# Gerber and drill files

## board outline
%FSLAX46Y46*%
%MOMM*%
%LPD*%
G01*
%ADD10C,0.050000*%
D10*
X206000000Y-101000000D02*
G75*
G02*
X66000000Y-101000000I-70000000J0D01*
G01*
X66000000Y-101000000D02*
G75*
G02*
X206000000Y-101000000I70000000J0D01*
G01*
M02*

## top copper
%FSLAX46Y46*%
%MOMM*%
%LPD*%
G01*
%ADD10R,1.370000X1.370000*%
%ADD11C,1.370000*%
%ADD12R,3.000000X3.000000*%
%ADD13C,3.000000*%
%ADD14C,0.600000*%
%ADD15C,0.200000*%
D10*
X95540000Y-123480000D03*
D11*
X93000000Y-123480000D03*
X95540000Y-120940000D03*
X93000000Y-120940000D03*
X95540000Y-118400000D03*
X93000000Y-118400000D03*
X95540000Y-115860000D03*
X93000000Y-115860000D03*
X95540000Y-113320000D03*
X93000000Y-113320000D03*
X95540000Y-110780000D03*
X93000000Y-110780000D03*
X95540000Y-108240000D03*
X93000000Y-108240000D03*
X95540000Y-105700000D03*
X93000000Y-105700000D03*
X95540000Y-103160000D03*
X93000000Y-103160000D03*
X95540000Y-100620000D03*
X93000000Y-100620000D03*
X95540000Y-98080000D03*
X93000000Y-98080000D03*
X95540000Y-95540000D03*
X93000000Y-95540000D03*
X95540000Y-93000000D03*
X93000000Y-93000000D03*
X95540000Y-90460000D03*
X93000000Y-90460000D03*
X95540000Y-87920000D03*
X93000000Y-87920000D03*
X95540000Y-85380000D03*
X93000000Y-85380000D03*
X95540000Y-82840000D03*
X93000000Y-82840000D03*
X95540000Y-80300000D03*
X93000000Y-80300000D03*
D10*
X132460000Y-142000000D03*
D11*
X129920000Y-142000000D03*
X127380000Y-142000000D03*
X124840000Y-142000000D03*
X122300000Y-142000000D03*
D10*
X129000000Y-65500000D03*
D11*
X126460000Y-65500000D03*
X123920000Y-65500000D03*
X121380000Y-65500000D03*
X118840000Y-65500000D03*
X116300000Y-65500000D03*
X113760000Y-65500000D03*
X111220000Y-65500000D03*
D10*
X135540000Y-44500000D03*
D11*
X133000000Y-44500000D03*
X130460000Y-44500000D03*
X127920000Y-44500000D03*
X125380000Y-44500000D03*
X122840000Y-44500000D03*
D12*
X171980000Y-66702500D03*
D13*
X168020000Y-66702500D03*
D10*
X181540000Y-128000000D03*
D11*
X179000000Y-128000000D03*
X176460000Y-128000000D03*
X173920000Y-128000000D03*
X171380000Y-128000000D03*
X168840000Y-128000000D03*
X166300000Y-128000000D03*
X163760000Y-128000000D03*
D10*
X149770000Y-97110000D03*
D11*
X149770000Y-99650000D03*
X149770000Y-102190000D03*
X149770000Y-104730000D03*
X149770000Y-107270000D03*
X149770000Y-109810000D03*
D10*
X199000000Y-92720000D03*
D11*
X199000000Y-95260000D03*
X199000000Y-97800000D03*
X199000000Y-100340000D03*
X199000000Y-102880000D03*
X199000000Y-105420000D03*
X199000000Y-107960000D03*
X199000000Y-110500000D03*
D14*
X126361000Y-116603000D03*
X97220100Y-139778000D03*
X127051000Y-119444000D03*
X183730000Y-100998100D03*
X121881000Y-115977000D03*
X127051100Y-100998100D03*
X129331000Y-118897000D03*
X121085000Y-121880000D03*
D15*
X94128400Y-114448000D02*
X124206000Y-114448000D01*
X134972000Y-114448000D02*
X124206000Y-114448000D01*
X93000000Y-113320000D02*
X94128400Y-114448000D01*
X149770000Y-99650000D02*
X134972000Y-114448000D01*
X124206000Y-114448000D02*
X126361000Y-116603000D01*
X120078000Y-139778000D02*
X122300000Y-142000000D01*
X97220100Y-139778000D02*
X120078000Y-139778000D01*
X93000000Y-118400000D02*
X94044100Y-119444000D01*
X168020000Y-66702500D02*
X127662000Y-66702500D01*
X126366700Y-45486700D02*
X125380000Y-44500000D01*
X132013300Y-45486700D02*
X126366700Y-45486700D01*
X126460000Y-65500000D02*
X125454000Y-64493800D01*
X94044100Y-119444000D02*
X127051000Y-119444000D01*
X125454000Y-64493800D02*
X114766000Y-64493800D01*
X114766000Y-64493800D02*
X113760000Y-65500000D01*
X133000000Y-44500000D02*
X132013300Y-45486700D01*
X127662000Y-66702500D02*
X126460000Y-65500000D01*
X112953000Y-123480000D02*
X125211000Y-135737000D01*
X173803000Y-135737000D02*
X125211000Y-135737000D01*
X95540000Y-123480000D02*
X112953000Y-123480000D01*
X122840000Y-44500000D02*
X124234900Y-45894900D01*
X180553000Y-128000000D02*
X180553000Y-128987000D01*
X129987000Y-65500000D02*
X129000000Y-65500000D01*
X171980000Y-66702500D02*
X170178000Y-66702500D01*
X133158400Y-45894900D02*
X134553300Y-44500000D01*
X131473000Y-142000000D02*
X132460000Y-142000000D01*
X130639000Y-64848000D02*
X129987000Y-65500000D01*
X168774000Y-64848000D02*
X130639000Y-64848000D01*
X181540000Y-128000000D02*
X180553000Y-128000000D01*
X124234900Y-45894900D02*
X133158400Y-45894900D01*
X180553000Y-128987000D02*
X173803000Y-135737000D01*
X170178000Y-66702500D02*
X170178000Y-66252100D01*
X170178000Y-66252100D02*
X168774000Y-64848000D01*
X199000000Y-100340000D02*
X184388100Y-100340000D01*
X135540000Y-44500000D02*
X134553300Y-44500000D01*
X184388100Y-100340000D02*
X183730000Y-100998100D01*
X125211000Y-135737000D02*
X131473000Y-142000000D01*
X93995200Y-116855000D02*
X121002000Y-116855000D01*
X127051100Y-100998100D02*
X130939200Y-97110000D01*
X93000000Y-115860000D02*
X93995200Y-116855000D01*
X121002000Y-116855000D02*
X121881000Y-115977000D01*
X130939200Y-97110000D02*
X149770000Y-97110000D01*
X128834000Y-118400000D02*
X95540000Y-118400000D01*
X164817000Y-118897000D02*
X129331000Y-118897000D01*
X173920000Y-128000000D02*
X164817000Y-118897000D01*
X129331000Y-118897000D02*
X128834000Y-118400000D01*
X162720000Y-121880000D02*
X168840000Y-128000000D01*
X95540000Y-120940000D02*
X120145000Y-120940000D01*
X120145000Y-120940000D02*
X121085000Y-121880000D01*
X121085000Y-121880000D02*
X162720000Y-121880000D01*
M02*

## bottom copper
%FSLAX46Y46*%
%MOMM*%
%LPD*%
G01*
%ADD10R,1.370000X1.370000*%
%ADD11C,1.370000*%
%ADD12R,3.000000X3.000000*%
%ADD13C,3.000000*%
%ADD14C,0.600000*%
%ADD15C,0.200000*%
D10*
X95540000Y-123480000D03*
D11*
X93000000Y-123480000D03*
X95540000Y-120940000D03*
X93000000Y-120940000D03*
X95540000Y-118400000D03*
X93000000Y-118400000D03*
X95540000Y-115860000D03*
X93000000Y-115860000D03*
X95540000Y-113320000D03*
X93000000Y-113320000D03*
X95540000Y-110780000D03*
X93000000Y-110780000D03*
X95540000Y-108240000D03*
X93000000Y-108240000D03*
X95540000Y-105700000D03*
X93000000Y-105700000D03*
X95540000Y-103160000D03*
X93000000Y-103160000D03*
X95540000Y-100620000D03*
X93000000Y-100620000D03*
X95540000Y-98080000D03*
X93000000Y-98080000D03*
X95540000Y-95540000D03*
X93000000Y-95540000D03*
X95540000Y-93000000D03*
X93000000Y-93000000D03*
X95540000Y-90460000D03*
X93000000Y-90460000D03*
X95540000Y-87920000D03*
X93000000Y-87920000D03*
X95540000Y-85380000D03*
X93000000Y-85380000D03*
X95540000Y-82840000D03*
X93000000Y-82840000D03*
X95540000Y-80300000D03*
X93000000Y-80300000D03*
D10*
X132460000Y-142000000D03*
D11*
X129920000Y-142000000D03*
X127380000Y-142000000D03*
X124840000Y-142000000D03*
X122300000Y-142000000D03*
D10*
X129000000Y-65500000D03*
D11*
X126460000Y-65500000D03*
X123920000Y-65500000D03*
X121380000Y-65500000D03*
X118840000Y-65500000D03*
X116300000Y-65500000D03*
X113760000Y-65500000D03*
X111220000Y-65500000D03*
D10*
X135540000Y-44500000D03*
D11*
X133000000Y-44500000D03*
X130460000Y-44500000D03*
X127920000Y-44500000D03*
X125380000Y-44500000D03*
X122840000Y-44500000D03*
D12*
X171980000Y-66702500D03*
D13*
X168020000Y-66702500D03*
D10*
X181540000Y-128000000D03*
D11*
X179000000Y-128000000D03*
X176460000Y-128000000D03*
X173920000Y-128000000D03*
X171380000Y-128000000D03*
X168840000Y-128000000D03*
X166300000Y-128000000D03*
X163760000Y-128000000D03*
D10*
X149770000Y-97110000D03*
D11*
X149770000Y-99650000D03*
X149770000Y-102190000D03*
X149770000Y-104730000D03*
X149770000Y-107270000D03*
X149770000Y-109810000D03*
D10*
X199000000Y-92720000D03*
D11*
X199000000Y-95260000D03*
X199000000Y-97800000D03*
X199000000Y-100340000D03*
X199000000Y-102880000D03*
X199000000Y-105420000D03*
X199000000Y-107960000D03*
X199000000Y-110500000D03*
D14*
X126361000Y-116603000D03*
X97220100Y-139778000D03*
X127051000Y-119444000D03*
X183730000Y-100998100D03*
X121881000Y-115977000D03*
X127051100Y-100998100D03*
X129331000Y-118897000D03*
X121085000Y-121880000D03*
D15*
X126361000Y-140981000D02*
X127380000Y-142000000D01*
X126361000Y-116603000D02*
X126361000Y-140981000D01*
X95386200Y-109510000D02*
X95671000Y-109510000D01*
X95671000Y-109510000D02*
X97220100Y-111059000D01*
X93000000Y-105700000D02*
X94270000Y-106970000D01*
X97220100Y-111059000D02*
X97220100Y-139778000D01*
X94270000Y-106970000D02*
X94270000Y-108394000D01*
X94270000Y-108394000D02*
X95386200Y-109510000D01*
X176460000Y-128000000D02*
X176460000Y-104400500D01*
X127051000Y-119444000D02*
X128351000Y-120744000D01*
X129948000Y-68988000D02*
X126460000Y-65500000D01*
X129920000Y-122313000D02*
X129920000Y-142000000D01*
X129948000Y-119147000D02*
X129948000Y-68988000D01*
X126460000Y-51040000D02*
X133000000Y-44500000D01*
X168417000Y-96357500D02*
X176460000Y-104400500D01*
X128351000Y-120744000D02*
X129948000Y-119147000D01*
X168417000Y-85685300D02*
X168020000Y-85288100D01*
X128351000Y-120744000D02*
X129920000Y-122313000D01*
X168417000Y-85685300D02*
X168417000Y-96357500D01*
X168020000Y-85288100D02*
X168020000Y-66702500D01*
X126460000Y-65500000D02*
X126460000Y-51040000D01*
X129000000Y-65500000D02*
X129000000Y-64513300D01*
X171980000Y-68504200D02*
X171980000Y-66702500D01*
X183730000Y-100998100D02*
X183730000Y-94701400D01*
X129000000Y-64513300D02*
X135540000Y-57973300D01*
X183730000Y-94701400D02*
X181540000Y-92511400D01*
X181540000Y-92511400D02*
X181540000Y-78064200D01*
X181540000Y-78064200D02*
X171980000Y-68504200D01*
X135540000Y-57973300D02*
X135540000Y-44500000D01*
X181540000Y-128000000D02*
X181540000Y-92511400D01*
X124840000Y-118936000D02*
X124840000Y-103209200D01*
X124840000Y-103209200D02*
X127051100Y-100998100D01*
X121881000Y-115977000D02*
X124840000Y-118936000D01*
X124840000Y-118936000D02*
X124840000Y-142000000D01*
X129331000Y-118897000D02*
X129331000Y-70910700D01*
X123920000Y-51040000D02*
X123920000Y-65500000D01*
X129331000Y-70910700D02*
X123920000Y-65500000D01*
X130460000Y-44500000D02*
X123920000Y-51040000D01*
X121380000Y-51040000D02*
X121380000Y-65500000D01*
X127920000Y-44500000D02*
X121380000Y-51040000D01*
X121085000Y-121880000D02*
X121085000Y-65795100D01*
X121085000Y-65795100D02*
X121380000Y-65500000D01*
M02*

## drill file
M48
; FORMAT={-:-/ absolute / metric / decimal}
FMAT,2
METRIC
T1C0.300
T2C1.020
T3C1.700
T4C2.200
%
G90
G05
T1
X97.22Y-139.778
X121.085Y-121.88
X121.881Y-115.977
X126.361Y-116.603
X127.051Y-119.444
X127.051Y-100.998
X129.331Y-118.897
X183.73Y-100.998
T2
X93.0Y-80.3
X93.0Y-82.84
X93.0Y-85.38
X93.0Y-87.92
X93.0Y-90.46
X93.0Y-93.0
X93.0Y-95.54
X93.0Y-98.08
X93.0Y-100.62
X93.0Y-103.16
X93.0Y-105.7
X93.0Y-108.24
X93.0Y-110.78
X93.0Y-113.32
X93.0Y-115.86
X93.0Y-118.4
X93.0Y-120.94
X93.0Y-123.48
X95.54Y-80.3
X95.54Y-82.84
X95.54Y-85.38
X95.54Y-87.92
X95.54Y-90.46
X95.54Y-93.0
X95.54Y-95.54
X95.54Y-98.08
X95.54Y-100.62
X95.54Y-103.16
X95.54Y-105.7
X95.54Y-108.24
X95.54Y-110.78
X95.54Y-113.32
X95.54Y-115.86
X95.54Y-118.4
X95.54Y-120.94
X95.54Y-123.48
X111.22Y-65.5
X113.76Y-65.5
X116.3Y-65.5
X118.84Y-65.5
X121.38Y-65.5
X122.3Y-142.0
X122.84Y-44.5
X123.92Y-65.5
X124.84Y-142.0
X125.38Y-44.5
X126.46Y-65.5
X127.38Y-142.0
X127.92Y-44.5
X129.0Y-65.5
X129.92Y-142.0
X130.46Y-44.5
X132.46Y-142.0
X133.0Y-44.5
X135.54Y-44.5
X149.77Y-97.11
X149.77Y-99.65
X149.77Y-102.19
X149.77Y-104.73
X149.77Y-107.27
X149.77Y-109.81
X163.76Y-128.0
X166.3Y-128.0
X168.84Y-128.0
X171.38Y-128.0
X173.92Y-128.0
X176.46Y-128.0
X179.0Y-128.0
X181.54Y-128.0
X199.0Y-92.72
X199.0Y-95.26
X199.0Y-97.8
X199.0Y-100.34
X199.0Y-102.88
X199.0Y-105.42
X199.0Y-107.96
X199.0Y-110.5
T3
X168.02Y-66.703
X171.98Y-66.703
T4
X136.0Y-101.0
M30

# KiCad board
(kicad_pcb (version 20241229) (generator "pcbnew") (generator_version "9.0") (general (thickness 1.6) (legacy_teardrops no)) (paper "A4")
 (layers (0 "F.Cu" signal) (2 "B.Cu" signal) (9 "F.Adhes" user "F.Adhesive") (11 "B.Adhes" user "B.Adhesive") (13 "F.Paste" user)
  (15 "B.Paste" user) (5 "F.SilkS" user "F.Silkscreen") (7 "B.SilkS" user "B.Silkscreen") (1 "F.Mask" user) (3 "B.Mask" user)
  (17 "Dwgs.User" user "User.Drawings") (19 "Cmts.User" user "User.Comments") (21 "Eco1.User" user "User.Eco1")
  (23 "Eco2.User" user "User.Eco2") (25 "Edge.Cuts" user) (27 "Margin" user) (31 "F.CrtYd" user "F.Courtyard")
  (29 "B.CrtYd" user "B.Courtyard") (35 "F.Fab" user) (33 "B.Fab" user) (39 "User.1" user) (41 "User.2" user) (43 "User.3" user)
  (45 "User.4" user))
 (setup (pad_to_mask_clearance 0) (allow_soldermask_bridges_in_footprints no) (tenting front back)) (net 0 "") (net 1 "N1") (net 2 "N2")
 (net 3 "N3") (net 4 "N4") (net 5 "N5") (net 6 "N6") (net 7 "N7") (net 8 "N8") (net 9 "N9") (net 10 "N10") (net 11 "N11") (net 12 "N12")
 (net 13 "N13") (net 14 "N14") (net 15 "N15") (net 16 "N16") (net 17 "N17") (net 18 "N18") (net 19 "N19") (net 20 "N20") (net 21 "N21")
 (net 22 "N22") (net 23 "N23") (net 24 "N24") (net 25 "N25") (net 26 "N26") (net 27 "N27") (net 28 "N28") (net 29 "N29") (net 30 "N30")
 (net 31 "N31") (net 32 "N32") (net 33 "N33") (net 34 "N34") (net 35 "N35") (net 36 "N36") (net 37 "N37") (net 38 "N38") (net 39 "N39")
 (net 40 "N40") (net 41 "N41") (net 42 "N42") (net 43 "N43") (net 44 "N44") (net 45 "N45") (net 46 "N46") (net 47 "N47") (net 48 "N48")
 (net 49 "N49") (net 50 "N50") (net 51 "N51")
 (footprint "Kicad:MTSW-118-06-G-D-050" (layer "F.Cu") (at 95.54 123.48 90)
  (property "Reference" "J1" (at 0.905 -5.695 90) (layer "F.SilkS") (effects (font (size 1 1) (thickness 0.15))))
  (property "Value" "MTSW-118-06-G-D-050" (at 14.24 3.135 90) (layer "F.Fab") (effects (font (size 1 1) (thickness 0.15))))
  (pad "01" thru_hole rect (at 0 0 90) (size 1.37 1.37) (drill 1.02) (layers "*.Cu" "*.Mask") (remove_unused_layers no) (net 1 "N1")
   (solder_mask_margin 0.102))
  (pad "02" thru_hole circle (at 0 -2.54 90) (size 1.37 1.37) (drill 1.02) (layers "*.Cu" "*.Mask") (remove_unused_layers no) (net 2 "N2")
   (solder_mask_margin 0.102))
  (pad "03" thru_hole circle (at 2.54 0 90) (size 1.37 1.37) (drill 1.02) (layers "*.Cu" "*.Mask") (remove_unused_layers no) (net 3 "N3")
   (solder_mask_margin 0.102))
  (pad "04" thru_hole circle (at 2.54 -2.54 90) (size 1.37 1.37) (drill 1.02) (layers "*.Cu" "*.Mask") (remove_unused_layers no)
   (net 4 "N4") (solder_mask_margin 0.102))
  (pad "05" thru_hole circle (at 5.08 0 90) (size 1.37 1.37) (drill 1.02) (layers "*.Cu" "*.Mask") (remove_unused_layers no) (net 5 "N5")
   (solder_mask_margin 0.102))
  (pad "06" thru_hole circle (at 5.08 -2.54 90) (size 1.37 1.37) (drill 1.02) (layers "*.Cu" "*.Mask") (remove_unused_layers no)
   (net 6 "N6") (solder_mask_margin 0.102))
  (pad "07" thru_hole circle (at 7.62 0 90) (size 1.37 1.37) (drill 1.02) (layers "*.Cu" "*.Mask") (remove_unused_layers no) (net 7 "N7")
   (solder_mask_margin 0.102))
  (pad "08" thru_hole circle (at 7.62 -2.54 90) (size 1.37 1.37) (drill 1.02) (layers "*.Cu" "*.Mask") (remove_unused_layers no)
   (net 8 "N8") (solder_mask_margin 0.102))
  (pad "09" thru_hole circle (at 10.16 0 90) (size 1.37 1.37) (drill 1.02) (layers "*.Cu" "*.Mask") (remove_unused_layers no) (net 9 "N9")
   (solder_mask_margin 0.102))
  (pad "10" thru_hole circle (at 10.16 -2.54 90) (size 1.37 1.37) (drill 1.02) (layers "*.Cu" "*.Mask") (remove_unused_layers no)
   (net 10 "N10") (solder_mask_margin 0.102))
  (pad "11" thru_hole circle (at 12.7 0 90) (size 1.37 1.37) (drill 1.02) (layers "*.Cu" "*.Mask") (remove_unused_layers no) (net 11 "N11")
   (solder_mask_margin 0.102))
  (pad "12" thru_hole circle (at 12.7 -2.54 90) (size 1.37 1.37) (drill 1.02) (layers "*.Cu" "*.Mask") (remove_unused_layers no)
   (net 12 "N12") (solder_mask_margin 0.102))
  (pad "13" thru_hole circle (at 15.24 0 90) (size 1.37 1.37) (drill 1.02) (layers "*.Cu" "*.Mask") (remove_unused_layers no) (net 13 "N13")
   (solder_mask_margin 0.102))
  (pad "14" thru_hole circle (at 15.24 -2.54 90) (size 1.37 1.37) (drill 1.02) (layers "*.Cu" "*.Mask") (remove_unused_layers no)
   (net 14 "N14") (solder_mask_margin 0.102))
  (pad "15" thru_hole circle (at 17.78 0 90) (size 1.37 1.37) (drill 1.02) (layers "*.Cu" "*.Mask") (remove_unused_layers no) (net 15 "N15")
   (solder_mask_margin 0.102))
  (pad "16" thru_hole circle (at 17.78 -2.54 90) (size 1.37 1.37) (drill 1.02) (layers "*.Cu" "*.Mask") (remove_unused_layers no)
   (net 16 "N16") (solder_mask_margin 0.102))
  (pad "17" thru_hole circle (at 20.32 0 90) (size 1.37 1.37) (drill 1.02) (layers "*.Cu" "*.Mask") (remove_unused_layers no) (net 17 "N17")
   (solder_mask_margin 0.102))
  (pad "18" thru_hole circle (at 20.32 -2.54 90) (size 1.37 1.37) (drill 1.02) (layers "*.Cu" "*.Mask") (remove_unused_layers no)
   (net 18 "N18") (solder_mask_margin 0.102))
  (pad "19" thru_hole circle (at 22.86 0 90) (size 1.37 1.37) (drill 1.02) (layers "*.Cu" "*.Mask") (remove_unused_layers no) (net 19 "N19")
   (solder_mask_margin 0.102))
  (pad "20" thru_hole circle (at 22.86 -2.54 90) (size 1.37 1.37) (drill 1.02) (layers "*.Cu" "*.Mask") (remove_unused_layers no)
   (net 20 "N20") (solder_mask_margin 0.102))
  (pad "21" thru_hole circle (at 25.4 0 90) (size 1.37 1.37) (drill 1.02) (layers "*.Cu" "*.Mask") (remove_unused_layers no) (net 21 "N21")
   (solder_mask_margin 0.102))
  (pad "22" thru_hole circle (at 25.4 -2.54 90) (size 1.37 1.37) (drill 1.02) (layers "*.Cu" "*.Mask") (remove_unused_layers no)
   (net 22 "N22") (solder_mask_margin 0.102))
  (pad "23" thru_hole circle (at 27.94 0 90) (size 1.37 1.37) (drill 1.02) (layers "*.Cu" "*.Mask") (remove_unused_layers no) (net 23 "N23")
   (solder_mask_margin 0.102))
  (pad "24" thru_hole circle (at 27.94 -2.54 90) (size 1.37 1.37) (drill 1.02) (layers "*.Cu" "*.Mask") (remove_unused_layers no)
   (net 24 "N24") (solder_mask_margin 0.102))
  (pad "25" thru_hole circle (at 30.48 0 90) (size 1.37 1.37) (drill 1.02) (layers "*.Cu" "*.Mask") (remove_unused_layers no) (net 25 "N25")
   (solder_mask_margin 0.102))
  (pad "26" thru_hole circle (at 30.48 -2.54 90) (size 1.37 1.37) (drill 1.02) (layers "*.Cu" "*.Mask") (remove_unused_layers no)
   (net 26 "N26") (solder_mask_margin 0.102))
  (pad "27" thru_hole circle (at 33.02 0 90) (size 1.37 1.37) (drill 1.02) (layers "*.Cu" "*.Mask") (remove_unused_layers no) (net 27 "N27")
   (solder_mask_margin 0.102))
  (pad "28" thru_hole circle (at 33.02 -2.54 90) (size 1.37 1.37) (drill 1.02) (layers "*.Cu" "*.Mask") (remove_unused_layers no)
   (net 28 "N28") (solder_mask_margin 0.102))
  (pad "29" thru_hole circle (at 35.56 0 90) (size 1.37 1.37) (drill 1.02) (layers "*.Cu" "*.Mask") (remove_unused_layers no) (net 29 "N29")
   (solder_mask_margin 0.102))
  (pad "30" thru_hole circle (at 35.56 -2.54 90) (size 1.37 1.37) (drill 1.02) (layers "*.Cu" "*.Mask") (remove_unused_layers no)
   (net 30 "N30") (solder_mask_margin 0.102))
  (pad "31" thru_hole circle (at 38.1 0 90) (size 1.37 1.37) (drill 1.02) (layers "*.Cu" "*.Mask") (remove_unused_layers no) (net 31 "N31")
   (solder_mask_margin 0.102))
  (pad "32" thru_hole circle (at 38.1 -2.54 90) (size 1.37 1.37) (drill 1.02) (layers "*.Cu" "*.Mask") (remove_unused_layers no)
   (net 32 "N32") (solder_mask_margin 0.102))
  (pad "33" thru_hole circle (at 40.64 0 90) (size 1.37 1.37) (drill 1.02) (layers "*.Cu" "*.Mask") (remove_unused_layers no) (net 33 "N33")
   (solder_mask_margin 0.102))
  (pad "34" thru_hole circle (at 40.64 -2.54 90) (size 1.37 1.37) (drill 1.02) (layers "*.Cu" "*.Mask") (remove_unused_layers no)
   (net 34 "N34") (solder_mask_margin 0.102))
  (pad "35" thru_hole circle (at 43.18 0 90) (size 1.37 1.37) (drill 1.02) (layers "*.Cu" "*.Mask") (remove_unused_layers no) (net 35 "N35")
   (solder_mask_margin 0.102))
  (pad "36" thru_hole circle (at 43.18 -2.54 90) (size 1.37 1.37) (drill 1.02) (layers "*.Cu" "*.Mask") (remove_unused_layers no)
   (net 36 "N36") (solder_mask_margin 0.102)))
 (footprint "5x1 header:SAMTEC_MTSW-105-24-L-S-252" (layer "F.Cu") (at 127.38 142)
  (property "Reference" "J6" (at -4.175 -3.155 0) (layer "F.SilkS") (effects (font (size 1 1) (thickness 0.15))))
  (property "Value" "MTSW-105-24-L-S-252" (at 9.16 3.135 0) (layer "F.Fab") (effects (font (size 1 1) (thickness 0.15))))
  (pad "01" thru_hole rect (at 5.08 0) (size 1.37 1.37) (drill 1.02) (layers "*.Cu" "*.Mask") (remove_unused_layers no) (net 1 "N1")
   (solder_mask_margin 0.102))
  (pad "02" thru_hole circle (at 2.54 0) (size 1.37 1.37) (drill 1.02) (layers "*.Cu" "*.Mask") (remove_unused_layers no) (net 6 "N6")
   (solder_mask_margin 0.102))
  (pad "03" thru_hole circle (at 0 0) (size 1.37 1.37) (drill 1.02) (layers "*.Cu" "*.Mask") (remove_unused_layers no) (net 10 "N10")
   (solder_mask_margin 0.102))
  (pad "04" thru_hole circle (at -2.54 0) (size 1.37 1.37) (drill 1.02) (layers "*.Cu" "*.Mask") (remove_unused_layers no) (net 8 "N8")
   (solder_mask_margin 0.102))
  (pad "05" thru_hole circle (at -5.08 0) (size 1.37 1.37) (drill 1.02) (layers "*.Cu" "*.Mask") (remove_unused_layers no) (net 16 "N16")
   (solder_mask_margin 0.102)))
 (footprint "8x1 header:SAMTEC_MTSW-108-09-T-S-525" (layer "F.Cu") (at 120.11 65.5)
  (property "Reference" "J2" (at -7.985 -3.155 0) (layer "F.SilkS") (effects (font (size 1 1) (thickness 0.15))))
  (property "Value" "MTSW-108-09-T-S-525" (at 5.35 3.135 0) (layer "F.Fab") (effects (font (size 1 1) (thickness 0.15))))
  (pad "01" thru_hole rect (at 8.89 0) (size 1.37 1.37) (drill 1.02) (layers "*.Cu" "*.Mask") (remove_unused_layers no) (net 1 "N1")
   (solder_mask_margin 0.102))
  (pad "02" thru_hole circle (at 6.35 0) (size 1.37 1.37) (drill 1.02) (layers "*.Cu" "*.Mask") (remove_unused_layers no) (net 6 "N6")
   (solder_mask_margin 0.102))
  (pad "03" thru_hole circle (at 3.81 0) (size 1.37 1.37) (drill 1.02) (layers "*.Cu" "*.Mask") (remove_unused_layers no) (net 5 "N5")
   (solder_mask_margin 0.102))
  (pad "04" thru_hole circle (at 1.27 0) (size 1.37 1.37) (drill 1.02) (layers "*.Cu" "*.Mask") (remove_unused_layers no) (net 3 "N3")
   (solder_mask_margin 0.102))
  (pad "05" thru_hole circle (at -1.27 0) (size 1.37 1.37) (drill 1.02) (layers "*.Cu" "*.Mask") (remove_unused_layers no) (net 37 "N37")
   (solder_mask_margin 0.102))
  (pad "06" thru_hole circle (at -3.81 0) (size 1.37 1.37) (drill 1.02) (layers "*.Cu" "*.Mask") (remove_unused_layers no) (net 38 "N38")
   (solder_mask_margin 0.102))
  (pad "07" thru_hole circle (at -6.35 0) (size 1.37 1.37) (drill 1.02) (layers "*.Cu" "*.Mask") (remove_unused_layers no) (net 6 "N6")
   (solder_mask_margin 0.102))
  (pad "08" thru_hole circle (at -8.89 0) (size 1.37 1.37) (drill 1.02) (layers "*.Cu" "*.Mask") (remove_unused_layers no) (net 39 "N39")
   (solder_mask_margin 0.102)))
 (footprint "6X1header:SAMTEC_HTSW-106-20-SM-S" (layer "F.Cu") (at 129.19 44.5)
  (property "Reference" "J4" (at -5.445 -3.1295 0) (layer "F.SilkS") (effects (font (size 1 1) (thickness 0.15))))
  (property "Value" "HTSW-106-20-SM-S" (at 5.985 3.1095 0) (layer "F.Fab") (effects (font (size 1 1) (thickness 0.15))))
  (pad "01" thru_hole rect (at 6.35 0) (size 1.37 1.37) (drill 1.02) (layers "*.Cu" "*.Mask") (remove_unused_layers no) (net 1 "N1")
   (solder_mask_margin 0.102))
  (pad "02" thru_hole circle (at 3.81 0) (size 1.37 1.37) (drill 1.02) (layers "*.Cu" "*.Mask") (remove_unused_layers no) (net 6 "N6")
   (solder_mask_margin 0.102))
  (pad "03" thru_hole circle (at 1.27 0) (size 1.37 1.37) (drill 1.02) (layers "*.Cu" "*.Mask") (remove_unused_layers no) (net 5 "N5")
   (solder_mask_margin 0.102))
  (pad "04" thru_hole circle (at -1.27 0) (size 1.37 1.37) (drill 1.02) (layers "*.Cu" "*.Mask") (remove_unused_layers no) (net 3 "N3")
   (solder_mask_margin 0.102))
  (pad "05" thru_hole circle (at -3.81 0) (size 1.37 1.37) (drill 1.02) (layers "*.Cu" "*.Mask") (remove_unused_layers no) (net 6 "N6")
   (solder_mask_margin 0.102))
  (pad "06" thru_hole circle (at -6.35 0) (size 1.37 1.37) (drill 1.02) (layers "*.Cu" "*.Mask") (remove_unused_layers no) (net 1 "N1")
   (solder_mask_margin 0.102)))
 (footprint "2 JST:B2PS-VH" (layer "F.Cu") (at 170 66.7025 180)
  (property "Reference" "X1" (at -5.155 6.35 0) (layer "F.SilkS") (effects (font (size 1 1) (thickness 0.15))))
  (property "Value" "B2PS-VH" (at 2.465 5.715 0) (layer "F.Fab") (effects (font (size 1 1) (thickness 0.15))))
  (pad "1" thru_hole rect (at -1.98 0 180) (size 3 3) (drill 1.7) (layers "*.Cu" "*.Mask") (remove_unused_layers no) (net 1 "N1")
   (solder_mask_margin 0.102))
  (pad "2" thru_hole circle (at 1.98 0 180) (size 3 3) (drill 1.7) (layers "*.Cu" "*.Mask") (remove_unused_layers no) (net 6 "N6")
   (solder_mask_margin 0.102)))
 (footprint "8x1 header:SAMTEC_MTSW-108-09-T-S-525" (layer "F.Cu") (at 172.65 128)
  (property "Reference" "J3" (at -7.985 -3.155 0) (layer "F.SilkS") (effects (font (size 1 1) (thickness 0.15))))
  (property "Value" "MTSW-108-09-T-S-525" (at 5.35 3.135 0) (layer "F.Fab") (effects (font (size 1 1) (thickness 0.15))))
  (pad "01" thru_hole rect (at 8.89 0) (size 1.37 1.37) (drill 1.02) (layers "*.Cu" "*.Mask") (remove_unused_layers no) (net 1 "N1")
   (solder_mask_margin 0.102))
  (pad "02" thru_hole circle (at 6.35 0) (size 1.37 1.37) (drill 1.02) (layers "*.Cu" "*.Mask") (remove_unused_layers no) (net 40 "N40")
   (solder_mask_margin 0.102))
  (pad "03" thru_hole circle (at 3.81 0) (size 1.37 1.37) (drill 1.02) (layers "*.Cu" "*.Mask") (remove_unused_layers no) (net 6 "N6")
   (solder_mask_margin 0.102))
  (pad "04" thru_hole circle (at 1.27 0) (size 1.37 1.37) (drill 1.02) (layers "*.Cu" "*.Mask") (remove_unused_layers no) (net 5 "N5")
   (solder_mask_margin 0.102))
  (pad "05" thru_hole circle (at -1.27 0) (size 1.37 1.37) (drill 1.02) (layers "*.Cu" "*.Mask") (remove_unused_layers no) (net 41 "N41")
   (solder_mask_margin 0.102))
  (pad "06" thru_hole circle (at -3.81 0) (size 1.37 1.37) (drill 1.02) (layers "*.Cu" "*.Mask") (remove_unused_layers no) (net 3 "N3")
   (solder_mask_margin 0.102))
  (pad "07" thru_hole circle (at -6.35 0) (size 1.37 1.37) (drill 1.02) (layers "*.Cu" "*.Mask") (remove_unused_layers no) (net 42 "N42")
   (solder_mask_margin 0.102))
  (pad "08" thru_hole circle (at -8.89 0) (size 1.37 1.37) (drill 1.02) (layers "*.Cu" "*.Mask") (remove_unused_layers no) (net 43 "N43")
   (solder_mask_margin 0.102)))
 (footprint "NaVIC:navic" (layer "F.Cu") (at 187.77 101.61)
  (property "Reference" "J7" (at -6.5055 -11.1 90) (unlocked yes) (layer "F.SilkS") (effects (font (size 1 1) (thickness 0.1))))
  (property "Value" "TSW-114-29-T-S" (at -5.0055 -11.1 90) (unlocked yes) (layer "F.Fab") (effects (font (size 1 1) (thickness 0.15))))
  (pad "01" thru_hole rect (at -38 -4.5 90) (size 1.37 1.37) (drill 1.02) (layers "*.Cu" "*.Mask") (remove_unused_layers no) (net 8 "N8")
   (solder_mask_margin 0.102))
  (pad "02" thru_hole circle (at -38 -1.96 90) (size 1.37 1.37) (drill 1.02) (layers "*.Cu" "*.Mask") (remove_unused_layers no)
   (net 10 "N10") (solder_mask_margin 0.102))
  (pad "03" thru_hole circle (at -38 0.58 90) (size 1.37 1.37) (drill 1.02) (layers "*.Cu" "*.Mask") (remove_unused_layers no)
   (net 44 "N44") (solder_mask_margin 0.102))
  (pad "04" thru_hole circle (at -38 3.12 90) (size 1.37 1.37) (drill 1.02) (layers "*.Cu" "*.Mask") (remove_unused_layers no)
   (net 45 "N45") (solder_mask_margin 0.102))
  (pad "05" thru_hole circle (at -38 5.66 90) (size 1.37 1.37) (drill 1.02) (layers "*.Cu" "*.Mask") (remove_unused_layers no)
   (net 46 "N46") (solder_mask_margin 0.102))
  (pad "06" thru_hole circle (at -38 8.2 90) (size 1.37 1.37) (drill 1.02) (layers "*.Cu" "*.Mask") (remove_unused_layers no) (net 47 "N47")
   (solder_mask_margin 0.102))
  (pad "7" thru_hole rect (at 11.23 -8.89 90) (size 1.37 1.37) (drill 1.02) (layers "*.Cu" "*.Mask") (remove_unused_layers no)
   (solder_mask_margin 0.102))
  (pad "8" thru_hole circle (at 11.23 -6.35 90) (size 1.37 1.37) (drill 1.02) (layers "*.Cu" "*.Mask") (remove_unused_layers no)
   (solder_mask_margin 0.102))
  (pad "9" thru_hole circle (at 11.23 -3.81 90) (size 1.37 1.37) (drill 1.02) (layers "*.Cu" "*.Mask") (remove_unused_layers no)
   (solder_mask_margin 0.102))
  (pad "10" thru_hole circle (at 11.23 -1.27 90) (size 1.37 1.37) (drill 1.02) (layers "*.Cu" "*.Mask") (remove_unused_layers no)
   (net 1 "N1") (solder_mask_margin 0.102))
  (pad "11" thru_hole circle (at 11.23 1.27 90) (size 1.37 1.37) (drill 1.02) (layers "*.Cu" "*.Mask") (remove_unused_layers no)
   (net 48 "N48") (solder_mask_margin 0.102))
  (pad "12" thru_hole circle (at 11.23 3.81 90) (size 1.37 1.37) (drill 1.02) (layers "*.Cu" "*.Mask") (remove_unused_layers no)
   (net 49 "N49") (solder_mask_margin 0.102))
  (pad "13" thru_hole circle (at 11.23 6.35 90) (size 1.37 1.37) (drill 1.02) (layers "*.Cu" "*.Mask") (remove_unused_layers no)
   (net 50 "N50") (solder_mask_margin 0.102))
  (pad "14" thru_hole circle (at 11.23 8.89 90) (size 1.37 1.37) (drill 1.02) (layers "*.Cu" "*.Mask") (remove_unused_layers no)
   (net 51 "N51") (solder_mask_margin 0.102)))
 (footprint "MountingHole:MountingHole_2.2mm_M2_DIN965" (layer "F.Cu") (at 136 101)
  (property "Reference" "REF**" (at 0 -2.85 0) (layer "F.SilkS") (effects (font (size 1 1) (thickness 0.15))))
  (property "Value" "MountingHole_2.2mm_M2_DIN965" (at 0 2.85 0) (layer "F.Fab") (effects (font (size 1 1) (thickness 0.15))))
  (pad "" np_thru_hole circle (at 0 0) (size 2.2 2.2) (drill 2.2) (layers "*.Cu" "*.Mask")))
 (gr_circle (center 136 101) (end 206 101) (stroke (width 0.05) (type solid)) (fill no) (layer "Edge.Cuts"))
 (segment (start 94.1284 114.448) (end 124.206 114.448) (width 0.2) (layer "F.Cu") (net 10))
 (segment (start 134.972 114.448) (end 124.206 114.448) (width 0.2) (layer "F.Cu") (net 10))
 (segment (start 93 113.32) (end 94.1284 114.448) (width 0.2) (layer "F.Cu") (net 10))
 (segment (start 149.77 99.65) (end 134.972 114.448) (width 0.2) (layer "F.Cu") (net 10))
 (segment (start 124.206 114.448) (end 126.361 116.603) (width 0.2) (layer "F.Cu") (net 10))
 (via (at 126.361 116.603) (size 0.6) (drill 0.3) (layers "F.Cu" "B.Cu") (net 10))
 (segment (start 126.361 140.981) (end 127.38 142) (width 0.2) (layer "B.Cu") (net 10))
 (segment (start 126.361 116.603) (end 126.361 140.981) (width 0.2) (layer "B.Cu") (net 10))
 (segment (start 120.078 139.778) (end 122.3 142) (width 0.2) (layer "F.Cu") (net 16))
 (segment (start 97.2201 139.778) (end 120.078 139.778) (width 0.2) (layer "F.Cu") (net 16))
 (via (at 97.2201 139.778) (size 0.6) (drill 0.3) (layers "F.Cu" "B.Cu") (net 16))
 (segment (start 95.3862 109.51) (end 95.671 109.51) (width 0.2) (layer "B.Cu") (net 16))
 (segment (start 95.671 109.51) (end 97.2201 111.059) (width 0.2) (layer "B.Cu") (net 16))
 (segment (start 93 105.7) (end 94.27 106.97) (width 0.2) (layer "B.Cu") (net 16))
 (segment (start 97.2201 111.059) (end 97.2201 139.778) (width 0.2) (layer "B.Cu") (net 16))
 (segment (start 94.27 106.97) (end 94.27 108.394) (width 0.2) (layer "B.Cu") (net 16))
 (segment (start 94.27 108.394) (end 95.3862 109.51) (width 0.2) (layer "B.Cu") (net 16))
 (segment (start 93 118.4) (end 94.0441 119.444) (width 0.2) (layer "F.Cu") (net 6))
 (segment (start 168.02 66.7025) (end 127.662 66.7025) (width 0.2) (layer "F.Cu") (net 6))
 (segment (start 126.3667 45.4867) (end 125.38 44.5) (width 0.2) (layer "F.Cu") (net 6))
 (segment (start 132.0133 45.4867) (end 126.3667 45.4867) (width 0.2) (layer "F.Cu") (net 6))
 (segment (start 126.46 65.5) (end 125.454 64.4938) (width 0.2) (layer "F.Cu") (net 6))
 (segment (start 94.0441 119.444) (end 127.051 119.444) (width 0.2) (layer "F.Cu") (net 6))
 (segment (start 125.454 64.4938) (end 114.766 64.4938) (width 0.2) (layer "F.Cu") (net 6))
 (segment (start 114.766 64.4938) (end 113.76 65.5) (width 0.2) (layer "F.Cu") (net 6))
 (segment (start 133 44.5) (end 132.0133 45.4867) (width 0.2) (layer "F.Cu") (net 6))
 (segment (start 127.662 66.7025) (end 126.46 65.5) (width 0.2) (layer "F.Cu") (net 6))
 (via (at 127.051 119.444) (size 0.6) (drill 0.3) (layers "F.Cu" "B.Cu") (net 6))
 (segment (start 176.46 128) (end 176.46 104.4005) (width 0.2) (layer "B.Cu") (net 6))
 (segment (start 127.051 119.444) (end 128.351 120.744) (width 0.2) (layer "B.Cu") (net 6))
 (segment (start 129.948 68.988) (end 126.46 65.5) (width 0.2) (layer "B.Cu") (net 6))
 (segment (start 129.92 122.313) (end 129.92 142) (width 0.2) (layer "B.Cu") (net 6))
 (segment (start 129.948 119.147) (end 129.948 68.988) (width 0.2) (layer "B.Cu") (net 6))
 (segment (start 126.46 51.04) (end 133 44.5) (width 0.2) (layer "B.Cu") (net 6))
 (segment (start 168.417 96.3575) (end 176.46 104.4005) (width 0.2) (layer "B.Cu") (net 6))
 (segment (start 128.351 120.744) (end 129.948 119.147) (width 0.2) (layer "B.Cu") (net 6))
 (segment (start 168.417 85.6853) (end 168.02 85.2881) (width 0.2) (layer "B.Cu") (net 6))
 (segment (start 128.351 120.744) (end 129.92 122.313) (width 0.2) (layer "B.Cu") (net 6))
 (segment (start 168.417 85.6853) (end 168.417 96.3575) (width 0.2) (layer "B.Cu") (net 6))
 (segment (start 168.02 85.2881) (end 168.02 66.7025) (width 0.2) (layer "B.Cu") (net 6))
 (segment (start 126.46 65.5) (end 126.46 51.04) (width 0.2) (layer "B.Cu") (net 6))
 (segment (start 112.953 123.48) (end 125.211 135.737) (width 0.2) (layer "F.Cu") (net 1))
 (segment (start 173.803 135.737) (end 125.211 135.737) (width 0.2) (layer "F.Cu") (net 1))
 (segment (start 95.54 123.48) (end 112.953 123.48) (width 0.2) (layer "F.Cu") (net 1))
 (segment (start 122.84 44.5) (end 124.2349 45.8949) (width 0.2) (layer "F.Cu") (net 1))
 (segment (start 180.553 128) (end 180.553 128.987) (width 0.2) (layer "F.Cu") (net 1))
 (segment (start 129.987 65.5) (end 129 65.5) (width 0.2) (layer "F.Cu") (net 1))
 (segment (start 171.98 66.7025) (end 170.178 66.7025) (width 0.2) (layer "F.Cu") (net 1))
 (segment (start 133.1584 45.8949) (end 134.5533 44.5) (width 0.2) (layer "F.Cu") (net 1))
 (segment (start 131.473 142) (end 132.46 142) (width 0.2) (layer "F.Cu") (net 1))
 (segment (start 130.639 64.848) (end 129.987 65.5) (width 0.2) (layer "F.Cu") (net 1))
 (segment (start 168.774 64.848) (end 130.639 64.848) (width 0.2) (layer "F.Cu") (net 1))
 (segment (start 181.54 128) (end 180.553 128) (width 0.2) (layer "F.Cu") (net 1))
 (segment (start 124.2349 45.8949) (end 133.1584 45.8949) (width 0.2) (layer "F.Cu") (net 1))
 (segment (start 180.553 128.987) (end 173.803 135.737) (width 0.2) (layer "F.Cu") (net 1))
 (segment (start 170.178 66.7025) (end 170.178 66.2521) (width 0.2) (layer "F.Cu") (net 1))
 (segment (start 170.178 66.2521) (end 168.774 64.848) (width 0.2) (layer "F.Cu") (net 1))
 (segment (start 199 100.34) (end 184.3881 100.34) (width 0.2) (layer "F.Cu") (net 1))
 (segment (start 135.54 44.5) (end 134.5533 44.5) (width 0.2) (layer "F.Cu") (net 1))
 (segment (start 184.3881 100.34) (end 183.73 100.9981) (width 0.2) (layer "F.Cu") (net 1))
 (segment (start 125.211 135.737) (end 131.473 142) (width 0.2) (layer "F.Cu") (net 1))
 (via (at 183.73 100.9981) (size 0.6) (drill 0.3) (layers "F.Cu" "B.Cu") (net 1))
 (segment (start 129 65.5) (end 129 64.5133) (width 0.2) (layer "B.Cu") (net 1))
 (segment (start 171.98 68.5042) (end 171.98 66.7025) (width 0.2) (layer "B.Cu") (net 1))
 (segment (start 183.73 100.9981) (end 183.73 94.7014) (width 0.2) (layer "B.Cu") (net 1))
 (segment (start 129 64.5133) (end 135.54 57.9733) (width 0.2) (layer "B.Cu") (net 1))
 (segment (start 183.73 94.7014) (end 181.54 92.5114) (width 0.2) (layer "B.Cu") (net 1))
 (segment (start 181.54 92.5114) (end 181.54 78.0642) (width 0.2) (layer "B.Cu") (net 1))
 (segment (start 181.54 78.0642) (end 171.98 68.5042) (width 0.2) (layer "B.Cu") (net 1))
 (segment (start 135.54 57.9733) (end 135.54 44.5) (width 0.2) (layer "B.Cu") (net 1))
 (segment (start 181.54 128) (end 181.54 92.5114) (width 0.2) (layer "B.Cu") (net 1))
 (segment (start 93.9952 116.855) (end 121.002 116.855) (width 0.2) (layer "F.Cu") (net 8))
 (segment (start 127.0511 100.9981) (end 130.9392 97.11) (width 0.2) (layer "F.Cu") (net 8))
 (segment (start 93 115.86) (end 93.9952 116.855) (width 0.2) (layer "F.Cu") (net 8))
 (segment (start 121.002 116.855) (end 121.881 115.977) (width 0.2) (layer "F.Cu") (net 8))
 (segment (start 130.9392 97.11) (end 149.77 97.11) (width 0.2) (layer "F.Cu") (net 8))
 (via (at 121.881 115.977) (size 0.6) (drill 0.3) (layers "F.Cu" "B.Cu") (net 8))
 (via (at 127.0511 100.9981) (size 0.6) (drill 0.3) (layers "F.Cu" "B.Cu") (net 8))
 (segment (start 124.84 118.936) (end 124.84 103.2092) (width 0.2) (layer "B.Cu") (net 8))
 (segment (start 124.84 103.2092) (end 127.0511 100.9981) (width 0.2) (layer "B.Cu") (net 8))
 (segment (start 121.881 115.977) (end 124.84 118.936) (width 0.2) (layer "B.Cu") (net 8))
 (segment (start 124.84 118.936) (end 124.84 142) (width 0.2) (layer "B.Cu") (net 8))
 (segment (start 128.834 118.4) (end 95.54 118.4) (width 0.2) (layer "F.Cu") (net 5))
 (segment (start 164.817 118.897) (end 129.331 118.897) (width 0.2) (layer "F.Cu") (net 5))
 (segment (start 173.92 128) (end 164.817 118.897) (width 0.2) (layer "F.Cu") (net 5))
 (segment (start 129.331 118.897) (end 128.834 118.4) (width 0.2) (layer "F.Cu") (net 5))
 (via (at 129.331 118.897) (size 0.6) (drill 0.3) (layers "F.Cu" "B.Cu") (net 5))
 (segment (start 129.331 118.897) (end 129.331 70.9107) (width 0.2) (layer "B.Cu") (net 5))
 (segment (start 123.92 51.04) (end 123.92 65.5) (width 0.2) (layer "B.Cu") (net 5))
 (segment (start 129.331 70.9107) (end 123.92 65.5) (width 0.2) (layer "B.Cu") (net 5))
 (segment (start 130.46 44.5) (end 123.92 51.04) (width 0.2) (layer "B.Cu") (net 5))
 (segment (start 162.72 121.88) (end 168.84 128) (width 0.2) (layer "F.Cu") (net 3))
 (segment (start 95.54 120.94) (end 120.145 120.94) (width 0.2) (layer "F.Cu") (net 3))
 (segment (start 120.145 120.94) (end 121.085 121.88) (width 0.2) (layer "F.Cu") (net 3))
 (segment (start 121.085 121.88) (end 162.72 121.88) (width 0.2) (layer "F.Cu") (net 3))
 (via (at 121.085 121.88) (size 0.6) (drill 0.3) (layers "F.Cu" "B.Cu") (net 3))
 (segment (start 121.38 51.04) (end 121.38 65.5) (width 0.2) (layer "B.Cu") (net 3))
 (segment (start 127.92 44.5) (end 121.38 51.04) (width 0.2) (layer "B.Cu") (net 3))
 (segment (start 121.085 121.88) (end 121.085 65.7951) (width 0.2) (layer "B.Cu") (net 3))
 (segment (start 121.085 65.7951) (end 121.38 65.5) (width 0.2) (layer "B.Cu") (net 3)))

